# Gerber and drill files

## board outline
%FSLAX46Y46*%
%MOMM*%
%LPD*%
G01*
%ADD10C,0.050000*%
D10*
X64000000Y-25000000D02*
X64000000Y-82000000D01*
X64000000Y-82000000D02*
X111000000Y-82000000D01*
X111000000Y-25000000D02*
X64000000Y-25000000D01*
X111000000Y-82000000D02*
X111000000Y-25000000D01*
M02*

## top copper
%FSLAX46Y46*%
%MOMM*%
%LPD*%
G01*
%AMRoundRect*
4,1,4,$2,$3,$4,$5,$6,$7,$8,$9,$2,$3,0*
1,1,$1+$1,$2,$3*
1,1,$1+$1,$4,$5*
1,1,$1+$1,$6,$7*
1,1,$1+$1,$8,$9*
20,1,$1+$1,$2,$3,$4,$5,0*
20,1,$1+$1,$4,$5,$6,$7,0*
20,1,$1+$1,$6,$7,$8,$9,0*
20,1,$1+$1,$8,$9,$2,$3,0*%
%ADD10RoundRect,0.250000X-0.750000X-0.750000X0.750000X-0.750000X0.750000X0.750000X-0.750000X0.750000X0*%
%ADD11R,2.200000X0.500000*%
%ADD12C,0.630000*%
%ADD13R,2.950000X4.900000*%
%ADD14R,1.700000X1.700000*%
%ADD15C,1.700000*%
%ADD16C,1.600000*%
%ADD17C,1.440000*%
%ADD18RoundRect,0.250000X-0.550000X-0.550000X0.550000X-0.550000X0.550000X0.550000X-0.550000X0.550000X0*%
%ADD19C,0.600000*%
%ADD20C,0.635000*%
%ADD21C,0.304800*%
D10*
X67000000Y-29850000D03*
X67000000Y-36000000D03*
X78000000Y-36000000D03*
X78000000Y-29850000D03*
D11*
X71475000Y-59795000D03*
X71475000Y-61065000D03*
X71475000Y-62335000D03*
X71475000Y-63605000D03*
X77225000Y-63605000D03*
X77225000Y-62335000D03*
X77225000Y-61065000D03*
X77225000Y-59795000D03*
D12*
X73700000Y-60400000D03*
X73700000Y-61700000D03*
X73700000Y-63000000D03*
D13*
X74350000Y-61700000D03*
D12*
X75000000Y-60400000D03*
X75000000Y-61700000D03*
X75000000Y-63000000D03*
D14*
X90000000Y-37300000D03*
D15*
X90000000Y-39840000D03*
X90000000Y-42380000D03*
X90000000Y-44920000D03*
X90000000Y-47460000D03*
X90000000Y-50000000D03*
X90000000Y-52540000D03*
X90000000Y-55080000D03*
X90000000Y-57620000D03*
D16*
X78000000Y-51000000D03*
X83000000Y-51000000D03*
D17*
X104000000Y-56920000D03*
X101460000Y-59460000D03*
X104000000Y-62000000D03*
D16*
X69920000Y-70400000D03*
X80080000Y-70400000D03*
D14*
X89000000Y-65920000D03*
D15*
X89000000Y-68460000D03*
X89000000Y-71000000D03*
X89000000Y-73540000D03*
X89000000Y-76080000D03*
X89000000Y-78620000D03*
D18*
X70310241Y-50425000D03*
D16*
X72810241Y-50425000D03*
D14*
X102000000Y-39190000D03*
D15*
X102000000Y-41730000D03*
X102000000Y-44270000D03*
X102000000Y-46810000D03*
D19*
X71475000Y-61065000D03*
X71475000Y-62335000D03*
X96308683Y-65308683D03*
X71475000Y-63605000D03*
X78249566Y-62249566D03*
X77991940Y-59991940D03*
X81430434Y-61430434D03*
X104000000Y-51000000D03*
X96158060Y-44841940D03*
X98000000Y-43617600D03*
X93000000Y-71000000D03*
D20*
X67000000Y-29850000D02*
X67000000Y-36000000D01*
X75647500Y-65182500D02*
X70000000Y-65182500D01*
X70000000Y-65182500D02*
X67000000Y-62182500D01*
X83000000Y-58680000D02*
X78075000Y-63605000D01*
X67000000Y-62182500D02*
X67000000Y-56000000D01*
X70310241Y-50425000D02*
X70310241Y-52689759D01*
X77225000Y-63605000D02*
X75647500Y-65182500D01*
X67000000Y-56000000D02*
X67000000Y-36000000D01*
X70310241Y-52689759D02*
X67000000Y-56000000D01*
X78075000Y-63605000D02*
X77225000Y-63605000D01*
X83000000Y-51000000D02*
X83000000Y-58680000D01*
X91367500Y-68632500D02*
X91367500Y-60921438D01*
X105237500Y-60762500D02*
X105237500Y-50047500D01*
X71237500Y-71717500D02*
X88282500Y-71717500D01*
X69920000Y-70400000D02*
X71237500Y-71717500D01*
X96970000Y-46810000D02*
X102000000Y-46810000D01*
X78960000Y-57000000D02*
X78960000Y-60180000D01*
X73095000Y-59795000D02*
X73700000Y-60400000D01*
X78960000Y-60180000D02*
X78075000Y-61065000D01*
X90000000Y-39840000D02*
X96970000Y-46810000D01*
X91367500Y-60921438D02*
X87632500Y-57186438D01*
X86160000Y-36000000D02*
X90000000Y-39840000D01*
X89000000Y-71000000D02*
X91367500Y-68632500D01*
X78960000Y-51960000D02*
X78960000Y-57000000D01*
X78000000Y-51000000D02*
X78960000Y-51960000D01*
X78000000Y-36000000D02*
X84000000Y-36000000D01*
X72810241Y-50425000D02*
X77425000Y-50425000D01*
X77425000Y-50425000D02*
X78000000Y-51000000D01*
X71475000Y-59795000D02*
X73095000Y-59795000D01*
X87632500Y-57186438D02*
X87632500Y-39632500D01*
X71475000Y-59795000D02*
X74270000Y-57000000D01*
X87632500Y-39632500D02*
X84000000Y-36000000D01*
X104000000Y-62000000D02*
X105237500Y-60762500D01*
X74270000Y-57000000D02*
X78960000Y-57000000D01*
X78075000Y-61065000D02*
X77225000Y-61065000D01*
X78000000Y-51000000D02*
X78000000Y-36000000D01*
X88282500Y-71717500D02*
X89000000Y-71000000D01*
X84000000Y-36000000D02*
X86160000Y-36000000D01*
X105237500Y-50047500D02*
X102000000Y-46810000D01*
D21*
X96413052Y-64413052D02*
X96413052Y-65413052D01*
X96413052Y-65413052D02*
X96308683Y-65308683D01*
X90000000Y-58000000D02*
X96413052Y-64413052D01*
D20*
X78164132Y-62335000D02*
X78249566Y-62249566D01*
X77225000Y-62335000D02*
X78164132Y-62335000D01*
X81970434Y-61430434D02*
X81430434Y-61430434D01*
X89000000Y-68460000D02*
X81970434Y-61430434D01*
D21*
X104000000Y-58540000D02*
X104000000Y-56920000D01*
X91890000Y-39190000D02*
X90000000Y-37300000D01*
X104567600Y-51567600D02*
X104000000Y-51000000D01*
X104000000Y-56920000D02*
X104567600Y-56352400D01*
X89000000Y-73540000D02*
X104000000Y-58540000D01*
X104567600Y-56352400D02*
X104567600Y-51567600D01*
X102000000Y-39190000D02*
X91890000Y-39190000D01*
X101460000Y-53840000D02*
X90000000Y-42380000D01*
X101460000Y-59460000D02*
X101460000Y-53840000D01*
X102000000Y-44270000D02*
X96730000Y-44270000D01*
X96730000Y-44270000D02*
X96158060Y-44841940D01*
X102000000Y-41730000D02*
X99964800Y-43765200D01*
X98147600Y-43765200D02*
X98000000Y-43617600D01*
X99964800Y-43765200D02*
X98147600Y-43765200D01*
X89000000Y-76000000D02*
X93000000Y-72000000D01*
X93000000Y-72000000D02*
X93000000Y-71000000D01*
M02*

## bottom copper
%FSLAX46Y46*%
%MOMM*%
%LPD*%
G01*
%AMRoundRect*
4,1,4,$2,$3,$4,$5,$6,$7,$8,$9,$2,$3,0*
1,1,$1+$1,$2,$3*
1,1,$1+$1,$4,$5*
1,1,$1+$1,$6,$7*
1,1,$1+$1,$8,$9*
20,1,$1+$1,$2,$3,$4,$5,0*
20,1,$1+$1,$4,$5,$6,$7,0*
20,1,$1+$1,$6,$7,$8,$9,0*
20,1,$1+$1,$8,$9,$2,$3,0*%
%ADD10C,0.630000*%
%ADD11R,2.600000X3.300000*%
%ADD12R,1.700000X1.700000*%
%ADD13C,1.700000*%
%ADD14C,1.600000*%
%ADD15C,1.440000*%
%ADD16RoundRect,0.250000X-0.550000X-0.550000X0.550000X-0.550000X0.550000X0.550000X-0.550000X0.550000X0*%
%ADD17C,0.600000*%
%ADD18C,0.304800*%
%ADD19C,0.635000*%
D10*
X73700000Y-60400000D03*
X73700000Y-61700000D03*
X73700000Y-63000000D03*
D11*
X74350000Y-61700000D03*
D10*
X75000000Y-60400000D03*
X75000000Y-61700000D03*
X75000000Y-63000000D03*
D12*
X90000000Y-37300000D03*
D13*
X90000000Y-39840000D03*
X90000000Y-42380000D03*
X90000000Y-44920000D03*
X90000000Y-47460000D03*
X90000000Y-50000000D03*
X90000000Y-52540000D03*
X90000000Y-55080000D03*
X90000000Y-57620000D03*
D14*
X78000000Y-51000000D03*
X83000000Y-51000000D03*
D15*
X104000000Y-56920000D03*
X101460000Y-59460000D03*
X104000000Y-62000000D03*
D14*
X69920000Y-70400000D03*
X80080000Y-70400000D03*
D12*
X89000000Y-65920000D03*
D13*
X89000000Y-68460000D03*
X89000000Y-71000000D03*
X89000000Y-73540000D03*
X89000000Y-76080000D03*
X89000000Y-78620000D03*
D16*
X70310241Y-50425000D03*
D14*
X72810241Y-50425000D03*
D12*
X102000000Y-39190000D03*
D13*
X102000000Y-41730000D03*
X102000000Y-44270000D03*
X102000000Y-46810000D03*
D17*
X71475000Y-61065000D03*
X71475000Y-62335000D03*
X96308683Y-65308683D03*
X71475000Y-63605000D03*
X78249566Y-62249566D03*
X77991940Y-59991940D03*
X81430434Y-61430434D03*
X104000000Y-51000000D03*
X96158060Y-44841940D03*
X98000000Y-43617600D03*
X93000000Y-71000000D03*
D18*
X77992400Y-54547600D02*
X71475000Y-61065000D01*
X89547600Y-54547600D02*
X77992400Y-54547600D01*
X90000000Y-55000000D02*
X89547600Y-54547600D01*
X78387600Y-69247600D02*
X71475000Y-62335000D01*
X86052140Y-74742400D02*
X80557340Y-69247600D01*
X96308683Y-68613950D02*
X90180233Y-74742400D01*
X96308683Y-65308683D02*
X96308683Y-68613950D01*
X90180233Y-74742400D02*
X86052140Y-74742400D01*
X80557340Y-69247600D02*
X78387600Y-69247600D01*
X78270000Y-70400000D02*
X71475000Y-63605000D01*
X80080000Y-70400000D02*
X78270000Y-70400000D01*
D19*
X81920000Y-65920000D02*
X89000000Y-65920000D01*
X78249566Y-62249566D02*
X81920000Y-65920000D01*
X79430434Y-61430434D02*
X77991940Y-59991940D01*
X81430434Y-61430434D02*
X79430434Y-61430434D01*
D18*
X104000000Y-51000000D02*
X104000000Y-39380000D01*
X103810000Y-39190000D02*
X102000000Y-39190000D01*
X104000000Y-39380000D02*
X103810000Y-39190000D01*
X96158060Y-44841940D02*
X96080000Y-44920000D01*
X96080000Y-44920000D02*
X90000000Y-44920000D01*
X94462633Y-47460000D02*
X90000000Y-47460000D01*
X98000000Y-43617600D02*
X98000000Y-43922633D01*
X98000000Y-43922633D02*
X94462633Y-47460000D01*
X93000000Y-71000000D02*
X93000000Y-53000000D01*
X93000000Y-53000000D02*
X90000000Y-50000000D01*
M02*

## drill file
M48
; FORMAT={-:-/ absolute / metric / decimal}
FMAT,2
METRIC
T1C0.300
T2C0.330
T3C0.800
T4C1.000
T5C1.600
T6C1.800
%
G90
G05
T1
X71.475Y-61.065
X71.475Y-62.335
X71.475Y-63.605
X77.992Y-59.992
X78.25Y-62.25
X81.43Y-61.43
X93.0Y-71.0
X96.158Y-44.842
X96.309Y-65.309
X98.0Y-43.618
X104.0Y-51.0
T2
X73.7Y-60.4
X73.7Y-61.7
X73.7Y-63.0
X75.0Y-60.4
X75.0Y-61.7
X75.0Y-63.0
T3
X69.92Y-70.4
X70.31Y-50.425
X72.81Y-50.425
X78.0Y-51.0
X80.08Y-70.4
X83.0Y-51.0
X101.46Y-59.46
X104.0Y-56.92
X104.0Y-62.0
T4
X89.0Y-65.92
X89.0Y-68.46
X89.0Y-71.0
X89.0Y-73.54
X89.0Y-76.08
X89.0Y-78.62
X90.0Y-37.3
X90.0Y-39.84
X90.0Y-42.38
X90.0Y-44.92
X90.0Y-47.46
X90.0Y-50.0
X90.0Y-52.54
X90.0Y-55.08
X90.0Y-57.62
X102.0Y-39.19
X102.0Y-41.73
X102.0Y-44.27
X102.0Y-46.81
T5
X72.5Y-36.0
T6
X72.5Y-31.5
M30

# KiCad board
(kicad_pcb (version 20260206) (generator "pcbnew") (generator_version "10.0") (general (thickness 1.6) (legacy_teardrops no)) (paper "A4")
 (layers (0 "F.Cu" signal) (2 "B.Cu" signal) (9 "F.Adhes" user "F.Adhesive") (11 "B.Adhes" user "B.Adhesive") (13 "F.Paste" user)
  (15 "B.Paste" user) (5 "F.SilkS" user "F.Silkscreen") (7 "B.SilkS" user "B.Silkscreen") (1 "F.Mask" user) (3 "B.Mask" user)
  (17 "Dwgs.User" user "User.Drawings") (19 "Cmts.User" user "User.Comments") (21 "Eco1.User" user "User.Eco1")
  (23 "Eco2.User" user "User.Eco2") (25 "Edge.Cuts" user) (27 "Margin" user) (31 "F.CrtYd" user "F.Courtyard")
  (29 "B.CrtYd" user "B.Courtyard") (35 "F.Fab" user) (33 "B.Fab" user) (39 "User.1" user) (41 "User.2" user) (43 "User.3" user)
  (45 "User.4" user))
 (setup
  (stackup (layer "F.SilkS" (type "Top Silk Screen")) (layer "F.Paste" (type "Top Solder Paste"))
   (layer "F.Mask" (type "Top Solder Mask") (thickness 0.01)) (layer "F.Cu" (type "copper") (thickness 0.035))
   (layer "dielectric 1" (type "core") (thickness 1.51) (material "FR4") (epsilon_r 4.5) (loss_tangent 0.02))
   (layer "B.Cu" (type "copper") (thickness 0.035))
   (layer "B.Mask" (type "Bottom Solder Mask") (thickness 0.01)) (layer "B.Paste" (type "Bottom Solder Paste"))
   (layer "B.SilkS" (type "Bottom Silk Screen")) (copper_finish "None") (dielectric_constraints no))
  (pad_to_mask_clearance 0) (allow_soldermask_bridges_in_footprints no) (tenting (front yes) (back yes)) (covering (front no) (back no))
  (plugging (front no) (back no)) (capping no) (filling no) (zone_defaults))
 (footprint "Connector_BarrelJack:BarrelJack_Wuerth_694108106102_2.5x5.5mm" (layer "F.Cu") (at 72.5 32.925)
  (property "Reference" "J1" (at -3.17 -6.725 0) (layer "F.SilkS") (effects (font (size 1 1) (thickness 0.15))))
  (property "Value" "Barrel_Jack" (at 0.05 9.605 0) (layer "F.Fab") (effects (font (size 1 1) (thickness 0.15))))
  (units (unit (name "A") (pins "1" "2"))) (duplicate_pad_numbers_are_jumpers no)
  (pad "" np_thru_hole circle (at 0 -1.425) (size 1.8 1.8) (drill 1.8) (layers "*.Cu" "*.Mask"))
  (pad "" np_thru_hole circle (at 0 3.075) (size 1.6 1.6) (drill 1.6) (layers "*.Cu" "*.Mask"))
  (pad "1" smd roundrect (at -5.5 -3.075) (size 2 2) (layers "F.Cu" "F.Mask" "F.Paste") (roundrect_rratio 0.125) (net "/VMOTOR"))
  (pad "1" smd roundrect (at -5.5 3.075) (size 2 2) (layers "F.Cu" "F.Mask" "F.Paste") (roundrect_rratio 0.125) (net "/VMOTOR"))
  (pad "2" smd roundrect (at 5.5 3.075) (size 2 2) (layers "F.Cu" "F.Mask" "F.Paste") (roundrect_rratio 0.125) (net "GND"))
  (pad "3" smd roundrect (at 5.5 -3.075) (size 2 2) (layers "F.Cu" "F.Mask" "F.Paste") (roundrect_rratio 0.125)))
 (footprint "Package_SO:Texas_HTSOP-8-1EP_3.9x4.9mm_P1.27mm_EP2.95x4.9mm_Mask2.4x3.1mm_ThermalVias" (layer "F.Cu") (at 74.35 61.7)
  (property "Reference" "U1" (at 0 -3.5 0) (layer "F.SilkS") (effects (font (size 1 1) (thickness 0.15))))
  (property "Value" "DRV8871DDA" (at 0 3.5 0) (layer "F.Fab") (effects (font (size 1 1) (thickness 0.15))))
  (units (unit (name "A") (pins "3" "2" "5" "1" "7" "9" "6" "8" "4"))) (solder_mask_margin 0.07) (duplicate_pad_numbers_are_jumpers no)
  (pad "" smd rect (at 0 0) (size 2.4 3.1) (layers "F.Mask")) (pad "" smd rect (at 0 0) (size 2.4 3.1) (layers "F.Paste"))
  (pad "1" smd rect (at -2.875 -1.905) (size 2.2 0.5) (layers "F.Cu" "F.Mask" "F.Paste") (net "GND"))
  (pad "2" smd rect (at -2.875 -0.635) (size 2.2 0.5) (layers "F.Cu" "F.Mask" "F.Paste") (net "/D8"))
  (pad "3" smd rect (at -2.875 0.635) (size 2.2 0.5) (layers "F.Cu" "F.Mask" "F.Paste") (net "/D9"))
  (pad "4" smd rect (at -2.875 1.905) (size 2.2 0.5) (layers "F.Cu" "F.Mask" "F.Paste") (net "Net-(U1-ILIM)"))
  (pad "5" smd rect (at 2.875 1.905) (size 2.2 0.5) (layers "F.Cu" "F.Mask" "F.Paste") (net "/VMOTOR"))
  (pad "6" smd rect (at 2.875 0.635) (size 2.2 0.5) (layers "F.Cu" "F.Mask" "F.Paste") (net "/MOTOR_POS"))
  (pad "7" smd rect (at 2.875 -0.635) (size 2.2 0.5) (layers "F.Cu" "F.Mask" "F.Paste") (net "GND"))
  (pad "8" smd rect (at 2.875 -1.905) (size 2.2 0.5) (layers "F.Cu" "F.Mask" "F.Paste") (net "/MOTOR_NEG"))
  (pad "9" thru_hole circle (at -0.65 -1.3) (size 0.63 0.63) (drill 0.33) (layers "*.Cu" "*.Mask") (remove_unused_layers no) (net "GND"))
  (pad "9" thru_hole circle (at -0.65 0) (size 0.63 0.63) (drill 0.33) (layers "*.Cu" "*.Mask") (remove_unused_layers no) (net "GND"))
  (pad "9" thru_hole circle (at -0.65 1.3) (size 0.63 0.63) (drill 0.33) (layers "*.Cu" "*.Mask") (remove_unused_layers no) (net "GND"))
  (pad "9" smd rect (at 0 0) (size 2.6 3.3) (layers "B.Cu") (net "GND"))
  (pad "9" smd rect (at 0 0) (size 2.95 4.9) (layers "F.Cu") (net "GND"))
  (pad "9" thru_hole circle (at 0.65 -1.3) (size 0.63 0.63) (drill 0.33) (layers "*.Cu" "*.Mask") (remove_unused_layers no) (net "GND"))
  (pad "9" thru_hole circle (at 0.65 0) (size 0.63 0.63) (drill 0.33) (layers "*.Cu" "*.Mask") (remove_unused_layers no) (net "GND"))
  (pad "9" thru_hole circle (at 0.65 1.3) (size 0.63 0.63) (drill 0.33) (layers "*.Cu" "*.Mask") (remove_unused_layers no) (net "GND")))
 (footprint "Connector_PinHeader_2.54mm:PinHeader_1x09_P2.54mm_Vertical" (layer "F.Cu") (at 90 37.3)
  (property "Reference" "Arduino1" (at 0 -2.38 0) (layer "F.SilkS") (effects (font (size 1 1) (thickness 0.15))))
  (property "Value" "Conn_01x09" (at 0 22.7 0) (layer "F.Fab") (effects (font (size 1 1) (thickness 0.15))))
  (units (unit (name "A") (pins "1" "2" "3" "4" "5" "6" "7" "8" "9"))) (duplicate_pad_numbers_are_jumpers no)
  (pad "1" thru_hole rect (at 0 0) (size 1.7 1.7) (drill 1) (layers "*.Cu" "*.Mask") (remove_unused_layers no) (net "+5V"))
  (pad "2" thru_hole circle (at 0 2.54) (size 1.7 1.7) (drill 1) (layers "*.Cu" "*.Mask") (remove_unused_layers no) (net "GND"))
  (pad "3" thru_hole circle (at 0 5.08) (size 1.7 1.7) (drill 1) (layers "*.Cu" "*.Mask") (remove_unused_layers no) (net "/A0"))
  (pad "4" thru_hole circle (at 0 7.62) (size 1.7 1.7) (drill 1) (layers "*.Cu" "*.Mask") (remove_unused_layers no) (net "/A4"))
  (pad "5" thru_hole circle (at 0 10.16) (size 1.7 1.7) (drill 1) (layers "*.Cu" "*.Mask") (remove_unused_layers no) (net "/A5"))
  (pad "6" thru_hole circle (at 0 12.7) (size 1.7 1.7) (drill 1) (layers "*.Cu" "*.Mask") (remove_unused_layers no) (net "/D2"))
  (pad "7" thru_hole circle (at 0 15.24) (size 1.7 1.7) (drill 1) (layers "*.Cu" "*.Mask") (remove_unused_layers no) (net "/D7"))
  (pad "8" thru_hole circle (at 0 17.78) (size 1.7 1.7) (drill 1) (layers "*.Cu" "*.Mask") (remove_unused_layers no) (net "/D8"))
  (pad "9" thru_hole circle (at 0 20.32) (size 1.7 1.7) (drill 1) (layers "*.Cu" "*.Mask") (remove_unused_layers no) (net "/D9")))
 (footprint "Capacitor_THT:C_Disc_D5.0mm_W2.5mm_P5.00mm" (layer "F.Cu") (at 78 51)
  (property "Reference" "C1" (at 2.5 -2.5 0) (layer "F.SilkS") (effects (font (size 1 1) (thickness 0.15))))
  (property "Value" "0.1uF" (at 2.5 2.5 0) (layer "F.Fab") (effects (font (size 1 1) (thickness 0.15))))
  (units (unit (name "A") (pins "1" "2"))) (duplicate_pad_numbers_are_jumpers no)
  (pad "1" thru_hole circle (at 0 0) (size 1.6 1.6) (drill 0.8) (layers "*.Cu" "*.Mask") (remove_unused_layers no) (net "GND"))
  (pad "2" thru_hole circle (at 5 0) (size 1.6 1.6) (drill 0.8) (layers "*.Cu" "*.Mask") (remove_unused_layers no) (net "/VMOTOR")))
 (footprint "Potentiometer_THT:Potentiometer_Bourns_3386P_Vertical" (layer "F.Cu") (at 104 56.92 180)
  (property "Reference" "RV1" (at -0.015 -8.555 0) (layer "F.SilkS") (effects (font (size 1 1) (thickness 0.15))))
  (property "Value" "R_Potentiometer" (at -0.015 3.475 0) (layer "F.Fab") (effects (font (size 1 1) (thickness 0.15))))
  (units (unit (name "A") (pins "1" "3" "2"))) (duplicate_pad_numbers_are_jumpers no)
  (pad "1" thru_hole circle (at 0 0 180) (size 1.44 1.44) (drill 0.8) (layers "*.Cu" "*.Mask") (remove_unused_layers no) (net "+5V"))
  (pad "2" thru_hole circle (at 2.54 -2.54 180) (size 1.44 1.44) (drill 0.8) (layers "*.Cu" "*.Mask") (remove_unused_layers no) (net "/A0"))
  (pad "3" thru_hole circle (at 0 -5.08 180) (size 1.44 1.44) (drill 0.8) (layers "*.Cu" "*.Mask") (remove_unused_layers no) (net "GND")))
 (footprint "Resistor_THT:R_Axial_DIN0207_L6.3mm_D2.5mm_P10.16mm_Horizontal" (layer "F.Cu") (at 69.92 70.4)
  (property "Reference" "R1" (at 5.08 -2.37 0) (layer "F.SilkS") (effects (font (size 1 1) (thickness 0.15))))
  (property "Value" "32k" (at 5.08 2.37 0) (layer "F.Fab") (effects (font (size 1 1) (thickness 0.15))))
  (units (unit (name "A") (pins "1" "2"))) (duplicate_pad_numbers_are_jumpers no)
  (pad "1" thru_hole circle (at 0 0) (size 1.6 1.6) (drill 0.8) (layers "*.Cu" "*.Mask") (remove_unused_layers no) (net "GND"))
  (pad "2" thru_hole circle (at 10.16 0) (size 1.6 1.6) (drill 0.8) (layers "*.Cu" "*.Mask") (remove_unused_layers no) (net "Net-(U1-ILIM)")))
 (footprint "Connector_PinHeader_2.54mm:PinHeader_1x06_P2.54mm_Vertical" (layer "F.Cu") (at 89 65.92)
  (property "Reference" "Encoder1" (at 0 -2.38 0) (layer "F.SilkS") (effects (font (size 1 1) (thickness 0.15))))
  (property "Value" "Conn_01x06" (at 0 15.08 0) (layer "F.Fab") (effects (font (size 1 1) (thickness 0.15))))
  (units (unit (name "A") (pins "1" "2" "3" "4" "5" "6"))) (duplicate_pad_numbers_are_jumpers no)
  (pad "1" thru_hole rect (at 0 0) (size 1.7 1.7) (drill 1) (layers "*.Cu" "*.Mask") (remove_unused_layers no) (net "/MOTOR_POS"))
  (pad "2" thru_hole circle (at 0 2.54) (size 1.7 1.7) (drill 1) (layers "*.Cu" "*.Mask") (remove_unused_layers no) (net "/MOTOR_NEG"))
  (pad "3" thru_hole circle (at 0 5.08) (size 1.7 1.7) (drill 1) (layers "*.Cu" "*.Mask") (remove_unused_layers no) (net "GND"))
  (pad "4" thru_hole circle (at 0 7.62) (size 1.7 1.7) (drill 1) (layers "*.Cu" "*.Mask") (remove_unused_layers no) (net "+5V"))
  (pad "5" thru_hole circle (at 0 10.16) (size 1.7 1.7) (drill 1) (layers "*.Cu" "*.Mask") (remove_unused_layers no) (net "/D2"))
  (pad "6" thru_hole circle (at 0 12.7) (size 1.7 1.7) (drill 1) (layers "*.Cu" "*.Mask") (remove_unused_layers no) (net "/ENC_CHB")))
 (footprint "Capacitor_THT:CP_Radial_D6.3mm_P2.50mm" (layer "F.Cu") (at 70.310241 50.425)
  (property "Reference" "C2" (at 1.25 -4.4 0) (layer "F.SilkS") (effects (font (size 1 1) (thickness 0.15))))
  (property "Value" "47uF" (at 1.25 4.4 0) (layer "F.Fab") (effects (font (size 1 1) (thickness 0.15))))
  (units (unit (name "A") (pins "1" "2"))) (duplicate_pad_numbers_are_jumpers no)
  (pad "1" thru_hole roundrect (at 0 0) (size 1.6 1.6) (drill 0.8) (layers "*.Cu" "*.Mask") (remove_unused_layers no)
   (roundrect_rratio 0.15625) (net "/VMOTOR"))
  (pad "2" thru_hole circle (at 2.5 0) (size 1.6 1.6) (drill 0.8) (layers "*.Cu" "*.Mask") (remove_unused_layers no) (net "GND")))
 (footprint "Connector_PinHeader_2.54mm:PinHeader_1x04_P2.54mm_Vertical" (layer "F.Cu") (at 102 39.19)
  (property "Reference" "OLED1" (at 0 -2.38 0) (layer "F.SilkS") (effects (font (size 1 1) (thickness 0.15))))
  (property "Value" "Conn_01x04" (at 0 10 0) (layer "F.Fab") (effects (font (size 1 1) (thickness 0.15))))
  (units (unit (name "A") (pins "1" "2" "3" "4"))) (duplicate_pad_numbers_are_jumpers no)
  (pad "1" thru_hole rect (at 0 0) (size 1.7 1.7) (drill 1) (layers "*.Cu" "*.Mask") (remove_unused_layers no) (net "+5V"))
  (pad "2" thru_hole circle (at 0 2.54) (size 1.7 1.7) (drill 1) (layers "*.Cu" "*.Mask") (remove_unused_layers no) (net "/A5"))
  (pad "3" thru_hole circle (at 0 5.08) (size 1.7 1.7) (drill 1) (layers "*.Cu" "*.Mask") (remove_unused_layers no) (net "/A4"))
  (pad "4" thru_hole circle (at 0 7.62) (size 1.7 1.7) (drill 1) (layers "*.Cu" "*.Mask") (remove_unused_layers no) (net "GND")))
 (gr_line (start 64 25) (end 64 82) (stroke (width 0.05) (type default)) (layer "Edge.Cuts"))
 (gr_line (start 64 82) (end 111 82) (stroke (width 0.05) (type default)) (layer "Edge.Cuts"))
 (gr_line (start 111 25) (end 64 25) (stroke (width 0.05) (type default)) (layer "Edge.Cuts"))
 (gr_line (start 111 82) (end 111 25) (stroke (width 0.05) (type default)) (layer "Edge.Cuts"))
 (segment (start 67 29.85) (end 67 36) (width 0.635) (layer "F.Cu") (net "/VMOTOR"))
 (segment (start 75.6475 65.1825) (end 70 65.1825) (width 0.635) (layer "F.Cu") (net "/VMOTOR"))
 (segment (start 70 65.1825) (end 67 62.1825) (width 0.635) (layer "F.Cu") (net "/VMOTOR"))
 (segment (start 83 58.68) (end 78.075 63.605) (width 0.635) (layer "F.Cu") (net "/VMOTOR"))
 (segment (start 67 62.1825) (end 67 56) (width 0.635) (layer "F.Cu") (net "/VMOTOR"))
 (segment (start 70.310241 50.425) (end 70.310241 52.689759) (width 0.635) (layer "F.Cu") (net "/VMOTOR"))
 (segment (start 77.225 63.605) (end 75.6475 65.1825) (width 0.635) (layer "F.Cu") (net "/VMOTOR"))
 (segment (start 67 56) (end 67 36) (width 0.635) (layer "F.Cu") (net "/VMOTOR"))
 (segment (start 70.310241 52.689759) (end 67 56) (width 0.635) (layer "F.Cu") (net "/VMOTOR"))
 (segment (start 78.075 63.605) (end 77.225 63.605) (width 0.635) (layer "F.Cu") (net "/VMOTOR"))
 (segment (start 83 51) (end 83 58.68) (width 0.635) (layer "F.Cu") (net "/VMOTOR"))
 (segment (start 91.3675 68.6325) (end 91.3675 60.921438) (width 0.635) (layer "F.Cu") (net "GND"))
 (segment (start 105.2375 60.7625) (end 105.2375 50.0475) (width 0.635) (layer "F.Cu") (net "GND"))
 (segment (start 71.2375 71.7175) (end 88.2825 71.7175) (width 0.635) (layer "F.Cu") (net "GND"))
 (segment (start 69.92 70.4) (end 71.2375 71.7175) (width 0.635) (layer "F.Cu") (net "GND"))
 (segment (start 96.97 46.81) (end 102 46.81) (width 0.635) (layer "F.Cu") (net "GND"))
 (segment (start 78.96 57) (end 78.96 60.18) (width 0.635) (layer "F.Cu") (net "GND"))
 (segment (start 73.095 59.795) (end 73.7 60.4) (width 0.635) (layer "F.Cu") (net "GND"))
 (segment (start 78.96 60.18) (end 78.075 61.065) (width 0.635) (layer "F.Cu") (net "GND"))
 (segment (start 90 39.84) (end 96.97 46.81) (width 0.635) (layer "F.Cu") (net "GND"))
 (segment (start 91.3675 60.921438) (end 87.6325 57.186438) (width 0.635) (layer "F.Cu") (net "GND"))
 (segment (start 86.16 36) (end 90 39.84) (width 0.635) (layer "F.Cu") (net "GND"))
 (segment (start 89 71) (end 91.3675 68.6325) (width 0.635) (layer "F.Cu") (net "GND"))
 (segment (start 78.96 51.96) (end 78.96 57) (width 0.635) (layer "F.Cu") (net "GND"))
 (segment (start 78 51) (end 78.96 51.96) (width 0.635) (layer "F.Cu") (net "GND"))
 (segment (start 78 36) (end 84 36) (width 0.635) (layer "F.Cu") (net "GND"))
 (segment (start 72.810241 50.425) (end 77.425 50.425) (width 0.635) (layer "F.Cu") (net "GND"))
 (segment (start 77.425 50.425) (end 78 51) (width 0.635) (layer "F.Cu") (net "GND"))
 (segment (start 71.475 59.795) (end 73.095 59.795) (width 0.635) (layer "F.Cu") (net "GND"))
 (segment (start 87.6325 57.186438) (end 87.6325 39.6325) (width 0.635) (layer "F.Cu") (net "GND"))
 (segment (start 71.475 59.795) (end 74.27 57) (width 0.635) (layer "F.Cu") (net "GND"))
 (segment (start 87.6325 39.6325) (end 84 36) (width 0.635) (layer "F.Cu") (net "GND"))
 (segment (start 104 62) (end 105.2375 60.7625) (width 0.635) (layer "F.Cu") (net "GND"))
 (segment (start 74.27 57) (end 78.96 57) (width 0.635) (layer "F.Cu") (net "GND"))
 (segment (start 78.075 61.065) (end 77.225 61.065) (width 0.635) (layer "F.Cu") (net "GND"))
 (segment (start 78 51) (end 78 36) (width 0.635) (layer "F.Cu") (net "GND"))
 (segment (start 88.2825 71.7175) (end 89 71) (width 0.635) (layer "F.Cu") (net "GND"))
 (segment (start 84 36) (end 86.16 36) (width 0.635) (layer "F.Cu") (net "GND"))
 (segment (start 105.2375 50.0475) (end 102 46.81) (width 0.635) (layer "F.Cu") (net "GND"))
 (via (at 71.475 61.065) (size 0.6) (drill 0.3) (layers "F.Cu" "B.Cu") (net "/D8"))
 (segment (start 77.9924 54.5476) (end 71.475 61.065) (width 0.3048) (layer "B.Cu") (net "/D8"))
 (segment (start 89.5476 54.5476) (end 77.9924 54.5476) (width 0.3048) (layer "B.Cu") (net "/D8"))
 (segment (start 90 55) (end 89.5476 54.5476) (width 0.3048) (layer "B.Cu") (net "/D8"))
 (segment (start 96.413052 64.413052) (end 96.413052 65.413052) (width 0.3048) (layer "F.Cu") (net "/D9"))
 (segment (start 96.413052 65.413052) (end 96.308683 65.308683) (width 0.3048) (layer "F.Cu") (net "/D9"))
 (segment (start 90 58) (end 96.413052 64.413052) (width 0.3048) (layer "F.Cu") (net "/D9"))
 (via (at 71.475 62.335) (size 0.6) (drill 0.3) (layers "F.Cu" "B.Cu") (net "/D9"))
 (via (at 96.308683 65.308683) (size 0.6) (drill 0.3) (layers "F.Cu" "B.Cu") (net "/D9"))
 (segment (start 78.3876 69.2476) (end 71.475 62.335) (width 0.3048) (layer "B.Cu") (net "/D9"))
 (segment (start 86.05214 74.7424) (end 80.55734 69.2476) (width 0.3048) (layer "B.Cu") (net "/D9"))
 (segment (start 96.308683 68.61395) (end 90.180233 74.7424) (width 0.3048) (layer "B.Cu") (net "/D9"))
 (segment (start 96.308683 65.308683) (end 96.308683 68.61395) (width 0.3048) (layer "B.Cu") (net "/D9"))
 (segment (start 90.180233 74.7424) (end 86.05214 74.7424) (width 0.3048) (layer "B.Cu") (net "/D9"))
 (segment (start 80.55734 69.2476) (end 78.3876 69.2476) (width 0.3048) (layer "B.Cu") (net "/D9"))
 (via (at 71.475 63.605) (size 0.6) (drill 0.3) (layers "F.Cu" "B.Cu") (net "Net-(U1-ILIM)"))
 (segment (start 78.27 70.4) (end 71.475 63.605) (width 0.3048) (layer "B.Cu") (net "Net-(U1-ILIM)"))
 (segment (start 80.08 70.4) (end 78.27 70.4) (width 0.3048) (layer "B.Cu") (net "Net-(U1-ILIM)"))
 (segment (start 78.164132 62.335) (end 78.249566 62.249566) (width 0.635) (layer "F.Cu") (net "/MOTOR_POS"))
 (segment (start 77.225 62.335) (end 78.164132 62.335) (width 0.635) (layer "F.Cu") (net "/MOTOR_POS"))
 (via (at 78.249566 62.249566) (size 0.6) (drill 0.3) (layers "F.Cu" "B.Cu") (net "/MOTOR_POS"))
 (segment (start 81.92 65.92) (end 89 65.92) (width 0.635) (layer "B.Cu") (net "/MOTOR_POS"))
 (segment (start 78.249566 62.249566) (end 81.92 65.92) (width 0.635) (layer "B.Cu") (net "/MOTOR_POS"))
 (segment (start 81.970434 61.430434) (end 81.430434 61.430434) (width 0.635) (layer "F.Cu") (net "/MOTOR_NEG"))
 (segment (start 89 68.46) (end 81.970434 61.430434) (width 0.635) (layer "F.Cu") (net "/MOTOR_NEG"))
 (via (at 77.99194 59.99194) (size 0.6) (drill 0.3) (layers "F.Cu" "B.Cu") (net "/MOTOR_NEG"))
 (via (at 81.430434 61.430434) (size 0.6) (drill 0.3) (layers "F.Cu" "B.Cu") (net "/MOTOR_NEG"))
 (segment (start 79.430434 61.430434) (end 77.99194 59.99194) (width 0.635) (layer "B.Cu") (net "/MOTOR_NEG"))
 (segment (start 81.430434 61.430434) (end 79.430434 61.430434) (width 0.635) (layer "B.Cu") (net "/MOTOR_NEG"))
 (segment (start 104 58.54) (end 104 56.92) (width 0.3048) (layer "F.Cu") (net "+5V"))
 (segment (start 91.89 39.19) (end 90 37.3) (width 0.3048) (layer "F.Cu") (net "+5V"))
 (segment (start 104.5676 51.5676) (end 104 51) (width 0.3048) (layer "F.Cu") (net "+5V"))
 (segment (start 104 56.92) (end 104.5676 56.3524) (width 0.3048) (layer "F.Cu") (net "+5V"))
 (segment (start 89 73.54) (end 104 58.54) (width 0.3048) (layer "F.Cu") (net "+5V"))
 (segment (start 104.5676 56.3524) (end 104.5676 51.5676) (width 0.3048) (layer "F.Cu") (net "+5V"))
 (segment (start 102 39.19) (end 91.89 39.19) (width 0.3048) (layer "F.Cu") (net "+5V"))
 (via (at 104 51) (size 0.6) (drill 0.3) (layers "F.Cu" "B.Cu") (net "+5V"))
 (segment (start 104 51) (end 104 39.38) (width 0.3048) (layer "B.Cu") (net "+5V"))
 (segment (start 103.81 39.19) (end 102 39.19) (width 0.3048) (layer "B.Cu") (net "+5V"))
 (segment (start 104 39.38) (end 103.81 39.19) (width 0.3048) (layer "B.Cu") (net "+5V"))
 (segment (start 101.46 53.84) (end 90 42.38) (width 0.3048) (layer "F.Cu") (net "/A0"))
 (segment (start 101.46 59.46) (end 101.46 53.84) (width 0.3048) (layer "F.Cu") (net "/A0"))
 (segment (start 102 44.27) (end 96.73 44.27) (width 0.3048) (layer "F.Cu") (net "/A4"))
 (segment (start 96.73 44.27) (end 96.15806 44.84194) (width 0.3048) (layer "F.Cu") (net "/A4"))
 (via (at 96.15806 44.84194) (size 0.6) (drill 0.3) (layers "F.Cu" "B.Cu") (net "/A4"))
 (segment (start 96.15806 44.84194) (end 96.08 44.92) (width 0.3048) (layer "B.Cu") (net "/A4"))
 (segment (start 96.08 44.92) (end 90 44.92) (width 0.3048) (layer "B.Cu") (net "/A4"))
 (segment (start 102 41.73) (end 99.9648 43.7652) (width 0.3048) (layer "F.Cu") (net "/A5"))
 (segment (start 98.1476 43.7652) (end 98 43.6176) (width 0.3048) (layer "F.Cu") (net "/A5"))
 (segment (start 99.9648 43.7652) (end 98.1476 43.7652) (width 0.3048) (layer "F.Cu") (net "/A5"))
 (via (at 98 43.6176) (size 0.6) (drill 0.3) (layers "F.Cu" "B.Cu") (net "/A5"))
 (segment (start 94.462633 47.46) (end 90 47.46) (width 0.3048) (layer "B.Cu") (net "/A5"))
 (segment (start 98 43.6176) (end 98 43.922633) (width 0.3048) (layer "B.Cu") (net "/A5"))
 (segment (start 98 43.922633) (end 94.462633 47.46) (width 0.3048) (layer "B.Cu") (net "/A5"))
 (segment (start 89 76) (end 93 72) (width 0.3048) (layer "F.Cu") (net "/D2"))
 (segment (start 93 72) (end 93 71) (width 0.3048) (layer "F.Cu") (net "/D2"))
 (via (at 93 71) (size 0.6) (drill 0.3) (layers "F.Cu" "B.Cu") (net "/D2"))
 (segment (start 93 71) (end 93 53) (width 0.3048) (layer "B.Cu") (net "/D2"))
 (segment (start 93 53) (end 90 50) (width 0.3048) (layer "B.Cu") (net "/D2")))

